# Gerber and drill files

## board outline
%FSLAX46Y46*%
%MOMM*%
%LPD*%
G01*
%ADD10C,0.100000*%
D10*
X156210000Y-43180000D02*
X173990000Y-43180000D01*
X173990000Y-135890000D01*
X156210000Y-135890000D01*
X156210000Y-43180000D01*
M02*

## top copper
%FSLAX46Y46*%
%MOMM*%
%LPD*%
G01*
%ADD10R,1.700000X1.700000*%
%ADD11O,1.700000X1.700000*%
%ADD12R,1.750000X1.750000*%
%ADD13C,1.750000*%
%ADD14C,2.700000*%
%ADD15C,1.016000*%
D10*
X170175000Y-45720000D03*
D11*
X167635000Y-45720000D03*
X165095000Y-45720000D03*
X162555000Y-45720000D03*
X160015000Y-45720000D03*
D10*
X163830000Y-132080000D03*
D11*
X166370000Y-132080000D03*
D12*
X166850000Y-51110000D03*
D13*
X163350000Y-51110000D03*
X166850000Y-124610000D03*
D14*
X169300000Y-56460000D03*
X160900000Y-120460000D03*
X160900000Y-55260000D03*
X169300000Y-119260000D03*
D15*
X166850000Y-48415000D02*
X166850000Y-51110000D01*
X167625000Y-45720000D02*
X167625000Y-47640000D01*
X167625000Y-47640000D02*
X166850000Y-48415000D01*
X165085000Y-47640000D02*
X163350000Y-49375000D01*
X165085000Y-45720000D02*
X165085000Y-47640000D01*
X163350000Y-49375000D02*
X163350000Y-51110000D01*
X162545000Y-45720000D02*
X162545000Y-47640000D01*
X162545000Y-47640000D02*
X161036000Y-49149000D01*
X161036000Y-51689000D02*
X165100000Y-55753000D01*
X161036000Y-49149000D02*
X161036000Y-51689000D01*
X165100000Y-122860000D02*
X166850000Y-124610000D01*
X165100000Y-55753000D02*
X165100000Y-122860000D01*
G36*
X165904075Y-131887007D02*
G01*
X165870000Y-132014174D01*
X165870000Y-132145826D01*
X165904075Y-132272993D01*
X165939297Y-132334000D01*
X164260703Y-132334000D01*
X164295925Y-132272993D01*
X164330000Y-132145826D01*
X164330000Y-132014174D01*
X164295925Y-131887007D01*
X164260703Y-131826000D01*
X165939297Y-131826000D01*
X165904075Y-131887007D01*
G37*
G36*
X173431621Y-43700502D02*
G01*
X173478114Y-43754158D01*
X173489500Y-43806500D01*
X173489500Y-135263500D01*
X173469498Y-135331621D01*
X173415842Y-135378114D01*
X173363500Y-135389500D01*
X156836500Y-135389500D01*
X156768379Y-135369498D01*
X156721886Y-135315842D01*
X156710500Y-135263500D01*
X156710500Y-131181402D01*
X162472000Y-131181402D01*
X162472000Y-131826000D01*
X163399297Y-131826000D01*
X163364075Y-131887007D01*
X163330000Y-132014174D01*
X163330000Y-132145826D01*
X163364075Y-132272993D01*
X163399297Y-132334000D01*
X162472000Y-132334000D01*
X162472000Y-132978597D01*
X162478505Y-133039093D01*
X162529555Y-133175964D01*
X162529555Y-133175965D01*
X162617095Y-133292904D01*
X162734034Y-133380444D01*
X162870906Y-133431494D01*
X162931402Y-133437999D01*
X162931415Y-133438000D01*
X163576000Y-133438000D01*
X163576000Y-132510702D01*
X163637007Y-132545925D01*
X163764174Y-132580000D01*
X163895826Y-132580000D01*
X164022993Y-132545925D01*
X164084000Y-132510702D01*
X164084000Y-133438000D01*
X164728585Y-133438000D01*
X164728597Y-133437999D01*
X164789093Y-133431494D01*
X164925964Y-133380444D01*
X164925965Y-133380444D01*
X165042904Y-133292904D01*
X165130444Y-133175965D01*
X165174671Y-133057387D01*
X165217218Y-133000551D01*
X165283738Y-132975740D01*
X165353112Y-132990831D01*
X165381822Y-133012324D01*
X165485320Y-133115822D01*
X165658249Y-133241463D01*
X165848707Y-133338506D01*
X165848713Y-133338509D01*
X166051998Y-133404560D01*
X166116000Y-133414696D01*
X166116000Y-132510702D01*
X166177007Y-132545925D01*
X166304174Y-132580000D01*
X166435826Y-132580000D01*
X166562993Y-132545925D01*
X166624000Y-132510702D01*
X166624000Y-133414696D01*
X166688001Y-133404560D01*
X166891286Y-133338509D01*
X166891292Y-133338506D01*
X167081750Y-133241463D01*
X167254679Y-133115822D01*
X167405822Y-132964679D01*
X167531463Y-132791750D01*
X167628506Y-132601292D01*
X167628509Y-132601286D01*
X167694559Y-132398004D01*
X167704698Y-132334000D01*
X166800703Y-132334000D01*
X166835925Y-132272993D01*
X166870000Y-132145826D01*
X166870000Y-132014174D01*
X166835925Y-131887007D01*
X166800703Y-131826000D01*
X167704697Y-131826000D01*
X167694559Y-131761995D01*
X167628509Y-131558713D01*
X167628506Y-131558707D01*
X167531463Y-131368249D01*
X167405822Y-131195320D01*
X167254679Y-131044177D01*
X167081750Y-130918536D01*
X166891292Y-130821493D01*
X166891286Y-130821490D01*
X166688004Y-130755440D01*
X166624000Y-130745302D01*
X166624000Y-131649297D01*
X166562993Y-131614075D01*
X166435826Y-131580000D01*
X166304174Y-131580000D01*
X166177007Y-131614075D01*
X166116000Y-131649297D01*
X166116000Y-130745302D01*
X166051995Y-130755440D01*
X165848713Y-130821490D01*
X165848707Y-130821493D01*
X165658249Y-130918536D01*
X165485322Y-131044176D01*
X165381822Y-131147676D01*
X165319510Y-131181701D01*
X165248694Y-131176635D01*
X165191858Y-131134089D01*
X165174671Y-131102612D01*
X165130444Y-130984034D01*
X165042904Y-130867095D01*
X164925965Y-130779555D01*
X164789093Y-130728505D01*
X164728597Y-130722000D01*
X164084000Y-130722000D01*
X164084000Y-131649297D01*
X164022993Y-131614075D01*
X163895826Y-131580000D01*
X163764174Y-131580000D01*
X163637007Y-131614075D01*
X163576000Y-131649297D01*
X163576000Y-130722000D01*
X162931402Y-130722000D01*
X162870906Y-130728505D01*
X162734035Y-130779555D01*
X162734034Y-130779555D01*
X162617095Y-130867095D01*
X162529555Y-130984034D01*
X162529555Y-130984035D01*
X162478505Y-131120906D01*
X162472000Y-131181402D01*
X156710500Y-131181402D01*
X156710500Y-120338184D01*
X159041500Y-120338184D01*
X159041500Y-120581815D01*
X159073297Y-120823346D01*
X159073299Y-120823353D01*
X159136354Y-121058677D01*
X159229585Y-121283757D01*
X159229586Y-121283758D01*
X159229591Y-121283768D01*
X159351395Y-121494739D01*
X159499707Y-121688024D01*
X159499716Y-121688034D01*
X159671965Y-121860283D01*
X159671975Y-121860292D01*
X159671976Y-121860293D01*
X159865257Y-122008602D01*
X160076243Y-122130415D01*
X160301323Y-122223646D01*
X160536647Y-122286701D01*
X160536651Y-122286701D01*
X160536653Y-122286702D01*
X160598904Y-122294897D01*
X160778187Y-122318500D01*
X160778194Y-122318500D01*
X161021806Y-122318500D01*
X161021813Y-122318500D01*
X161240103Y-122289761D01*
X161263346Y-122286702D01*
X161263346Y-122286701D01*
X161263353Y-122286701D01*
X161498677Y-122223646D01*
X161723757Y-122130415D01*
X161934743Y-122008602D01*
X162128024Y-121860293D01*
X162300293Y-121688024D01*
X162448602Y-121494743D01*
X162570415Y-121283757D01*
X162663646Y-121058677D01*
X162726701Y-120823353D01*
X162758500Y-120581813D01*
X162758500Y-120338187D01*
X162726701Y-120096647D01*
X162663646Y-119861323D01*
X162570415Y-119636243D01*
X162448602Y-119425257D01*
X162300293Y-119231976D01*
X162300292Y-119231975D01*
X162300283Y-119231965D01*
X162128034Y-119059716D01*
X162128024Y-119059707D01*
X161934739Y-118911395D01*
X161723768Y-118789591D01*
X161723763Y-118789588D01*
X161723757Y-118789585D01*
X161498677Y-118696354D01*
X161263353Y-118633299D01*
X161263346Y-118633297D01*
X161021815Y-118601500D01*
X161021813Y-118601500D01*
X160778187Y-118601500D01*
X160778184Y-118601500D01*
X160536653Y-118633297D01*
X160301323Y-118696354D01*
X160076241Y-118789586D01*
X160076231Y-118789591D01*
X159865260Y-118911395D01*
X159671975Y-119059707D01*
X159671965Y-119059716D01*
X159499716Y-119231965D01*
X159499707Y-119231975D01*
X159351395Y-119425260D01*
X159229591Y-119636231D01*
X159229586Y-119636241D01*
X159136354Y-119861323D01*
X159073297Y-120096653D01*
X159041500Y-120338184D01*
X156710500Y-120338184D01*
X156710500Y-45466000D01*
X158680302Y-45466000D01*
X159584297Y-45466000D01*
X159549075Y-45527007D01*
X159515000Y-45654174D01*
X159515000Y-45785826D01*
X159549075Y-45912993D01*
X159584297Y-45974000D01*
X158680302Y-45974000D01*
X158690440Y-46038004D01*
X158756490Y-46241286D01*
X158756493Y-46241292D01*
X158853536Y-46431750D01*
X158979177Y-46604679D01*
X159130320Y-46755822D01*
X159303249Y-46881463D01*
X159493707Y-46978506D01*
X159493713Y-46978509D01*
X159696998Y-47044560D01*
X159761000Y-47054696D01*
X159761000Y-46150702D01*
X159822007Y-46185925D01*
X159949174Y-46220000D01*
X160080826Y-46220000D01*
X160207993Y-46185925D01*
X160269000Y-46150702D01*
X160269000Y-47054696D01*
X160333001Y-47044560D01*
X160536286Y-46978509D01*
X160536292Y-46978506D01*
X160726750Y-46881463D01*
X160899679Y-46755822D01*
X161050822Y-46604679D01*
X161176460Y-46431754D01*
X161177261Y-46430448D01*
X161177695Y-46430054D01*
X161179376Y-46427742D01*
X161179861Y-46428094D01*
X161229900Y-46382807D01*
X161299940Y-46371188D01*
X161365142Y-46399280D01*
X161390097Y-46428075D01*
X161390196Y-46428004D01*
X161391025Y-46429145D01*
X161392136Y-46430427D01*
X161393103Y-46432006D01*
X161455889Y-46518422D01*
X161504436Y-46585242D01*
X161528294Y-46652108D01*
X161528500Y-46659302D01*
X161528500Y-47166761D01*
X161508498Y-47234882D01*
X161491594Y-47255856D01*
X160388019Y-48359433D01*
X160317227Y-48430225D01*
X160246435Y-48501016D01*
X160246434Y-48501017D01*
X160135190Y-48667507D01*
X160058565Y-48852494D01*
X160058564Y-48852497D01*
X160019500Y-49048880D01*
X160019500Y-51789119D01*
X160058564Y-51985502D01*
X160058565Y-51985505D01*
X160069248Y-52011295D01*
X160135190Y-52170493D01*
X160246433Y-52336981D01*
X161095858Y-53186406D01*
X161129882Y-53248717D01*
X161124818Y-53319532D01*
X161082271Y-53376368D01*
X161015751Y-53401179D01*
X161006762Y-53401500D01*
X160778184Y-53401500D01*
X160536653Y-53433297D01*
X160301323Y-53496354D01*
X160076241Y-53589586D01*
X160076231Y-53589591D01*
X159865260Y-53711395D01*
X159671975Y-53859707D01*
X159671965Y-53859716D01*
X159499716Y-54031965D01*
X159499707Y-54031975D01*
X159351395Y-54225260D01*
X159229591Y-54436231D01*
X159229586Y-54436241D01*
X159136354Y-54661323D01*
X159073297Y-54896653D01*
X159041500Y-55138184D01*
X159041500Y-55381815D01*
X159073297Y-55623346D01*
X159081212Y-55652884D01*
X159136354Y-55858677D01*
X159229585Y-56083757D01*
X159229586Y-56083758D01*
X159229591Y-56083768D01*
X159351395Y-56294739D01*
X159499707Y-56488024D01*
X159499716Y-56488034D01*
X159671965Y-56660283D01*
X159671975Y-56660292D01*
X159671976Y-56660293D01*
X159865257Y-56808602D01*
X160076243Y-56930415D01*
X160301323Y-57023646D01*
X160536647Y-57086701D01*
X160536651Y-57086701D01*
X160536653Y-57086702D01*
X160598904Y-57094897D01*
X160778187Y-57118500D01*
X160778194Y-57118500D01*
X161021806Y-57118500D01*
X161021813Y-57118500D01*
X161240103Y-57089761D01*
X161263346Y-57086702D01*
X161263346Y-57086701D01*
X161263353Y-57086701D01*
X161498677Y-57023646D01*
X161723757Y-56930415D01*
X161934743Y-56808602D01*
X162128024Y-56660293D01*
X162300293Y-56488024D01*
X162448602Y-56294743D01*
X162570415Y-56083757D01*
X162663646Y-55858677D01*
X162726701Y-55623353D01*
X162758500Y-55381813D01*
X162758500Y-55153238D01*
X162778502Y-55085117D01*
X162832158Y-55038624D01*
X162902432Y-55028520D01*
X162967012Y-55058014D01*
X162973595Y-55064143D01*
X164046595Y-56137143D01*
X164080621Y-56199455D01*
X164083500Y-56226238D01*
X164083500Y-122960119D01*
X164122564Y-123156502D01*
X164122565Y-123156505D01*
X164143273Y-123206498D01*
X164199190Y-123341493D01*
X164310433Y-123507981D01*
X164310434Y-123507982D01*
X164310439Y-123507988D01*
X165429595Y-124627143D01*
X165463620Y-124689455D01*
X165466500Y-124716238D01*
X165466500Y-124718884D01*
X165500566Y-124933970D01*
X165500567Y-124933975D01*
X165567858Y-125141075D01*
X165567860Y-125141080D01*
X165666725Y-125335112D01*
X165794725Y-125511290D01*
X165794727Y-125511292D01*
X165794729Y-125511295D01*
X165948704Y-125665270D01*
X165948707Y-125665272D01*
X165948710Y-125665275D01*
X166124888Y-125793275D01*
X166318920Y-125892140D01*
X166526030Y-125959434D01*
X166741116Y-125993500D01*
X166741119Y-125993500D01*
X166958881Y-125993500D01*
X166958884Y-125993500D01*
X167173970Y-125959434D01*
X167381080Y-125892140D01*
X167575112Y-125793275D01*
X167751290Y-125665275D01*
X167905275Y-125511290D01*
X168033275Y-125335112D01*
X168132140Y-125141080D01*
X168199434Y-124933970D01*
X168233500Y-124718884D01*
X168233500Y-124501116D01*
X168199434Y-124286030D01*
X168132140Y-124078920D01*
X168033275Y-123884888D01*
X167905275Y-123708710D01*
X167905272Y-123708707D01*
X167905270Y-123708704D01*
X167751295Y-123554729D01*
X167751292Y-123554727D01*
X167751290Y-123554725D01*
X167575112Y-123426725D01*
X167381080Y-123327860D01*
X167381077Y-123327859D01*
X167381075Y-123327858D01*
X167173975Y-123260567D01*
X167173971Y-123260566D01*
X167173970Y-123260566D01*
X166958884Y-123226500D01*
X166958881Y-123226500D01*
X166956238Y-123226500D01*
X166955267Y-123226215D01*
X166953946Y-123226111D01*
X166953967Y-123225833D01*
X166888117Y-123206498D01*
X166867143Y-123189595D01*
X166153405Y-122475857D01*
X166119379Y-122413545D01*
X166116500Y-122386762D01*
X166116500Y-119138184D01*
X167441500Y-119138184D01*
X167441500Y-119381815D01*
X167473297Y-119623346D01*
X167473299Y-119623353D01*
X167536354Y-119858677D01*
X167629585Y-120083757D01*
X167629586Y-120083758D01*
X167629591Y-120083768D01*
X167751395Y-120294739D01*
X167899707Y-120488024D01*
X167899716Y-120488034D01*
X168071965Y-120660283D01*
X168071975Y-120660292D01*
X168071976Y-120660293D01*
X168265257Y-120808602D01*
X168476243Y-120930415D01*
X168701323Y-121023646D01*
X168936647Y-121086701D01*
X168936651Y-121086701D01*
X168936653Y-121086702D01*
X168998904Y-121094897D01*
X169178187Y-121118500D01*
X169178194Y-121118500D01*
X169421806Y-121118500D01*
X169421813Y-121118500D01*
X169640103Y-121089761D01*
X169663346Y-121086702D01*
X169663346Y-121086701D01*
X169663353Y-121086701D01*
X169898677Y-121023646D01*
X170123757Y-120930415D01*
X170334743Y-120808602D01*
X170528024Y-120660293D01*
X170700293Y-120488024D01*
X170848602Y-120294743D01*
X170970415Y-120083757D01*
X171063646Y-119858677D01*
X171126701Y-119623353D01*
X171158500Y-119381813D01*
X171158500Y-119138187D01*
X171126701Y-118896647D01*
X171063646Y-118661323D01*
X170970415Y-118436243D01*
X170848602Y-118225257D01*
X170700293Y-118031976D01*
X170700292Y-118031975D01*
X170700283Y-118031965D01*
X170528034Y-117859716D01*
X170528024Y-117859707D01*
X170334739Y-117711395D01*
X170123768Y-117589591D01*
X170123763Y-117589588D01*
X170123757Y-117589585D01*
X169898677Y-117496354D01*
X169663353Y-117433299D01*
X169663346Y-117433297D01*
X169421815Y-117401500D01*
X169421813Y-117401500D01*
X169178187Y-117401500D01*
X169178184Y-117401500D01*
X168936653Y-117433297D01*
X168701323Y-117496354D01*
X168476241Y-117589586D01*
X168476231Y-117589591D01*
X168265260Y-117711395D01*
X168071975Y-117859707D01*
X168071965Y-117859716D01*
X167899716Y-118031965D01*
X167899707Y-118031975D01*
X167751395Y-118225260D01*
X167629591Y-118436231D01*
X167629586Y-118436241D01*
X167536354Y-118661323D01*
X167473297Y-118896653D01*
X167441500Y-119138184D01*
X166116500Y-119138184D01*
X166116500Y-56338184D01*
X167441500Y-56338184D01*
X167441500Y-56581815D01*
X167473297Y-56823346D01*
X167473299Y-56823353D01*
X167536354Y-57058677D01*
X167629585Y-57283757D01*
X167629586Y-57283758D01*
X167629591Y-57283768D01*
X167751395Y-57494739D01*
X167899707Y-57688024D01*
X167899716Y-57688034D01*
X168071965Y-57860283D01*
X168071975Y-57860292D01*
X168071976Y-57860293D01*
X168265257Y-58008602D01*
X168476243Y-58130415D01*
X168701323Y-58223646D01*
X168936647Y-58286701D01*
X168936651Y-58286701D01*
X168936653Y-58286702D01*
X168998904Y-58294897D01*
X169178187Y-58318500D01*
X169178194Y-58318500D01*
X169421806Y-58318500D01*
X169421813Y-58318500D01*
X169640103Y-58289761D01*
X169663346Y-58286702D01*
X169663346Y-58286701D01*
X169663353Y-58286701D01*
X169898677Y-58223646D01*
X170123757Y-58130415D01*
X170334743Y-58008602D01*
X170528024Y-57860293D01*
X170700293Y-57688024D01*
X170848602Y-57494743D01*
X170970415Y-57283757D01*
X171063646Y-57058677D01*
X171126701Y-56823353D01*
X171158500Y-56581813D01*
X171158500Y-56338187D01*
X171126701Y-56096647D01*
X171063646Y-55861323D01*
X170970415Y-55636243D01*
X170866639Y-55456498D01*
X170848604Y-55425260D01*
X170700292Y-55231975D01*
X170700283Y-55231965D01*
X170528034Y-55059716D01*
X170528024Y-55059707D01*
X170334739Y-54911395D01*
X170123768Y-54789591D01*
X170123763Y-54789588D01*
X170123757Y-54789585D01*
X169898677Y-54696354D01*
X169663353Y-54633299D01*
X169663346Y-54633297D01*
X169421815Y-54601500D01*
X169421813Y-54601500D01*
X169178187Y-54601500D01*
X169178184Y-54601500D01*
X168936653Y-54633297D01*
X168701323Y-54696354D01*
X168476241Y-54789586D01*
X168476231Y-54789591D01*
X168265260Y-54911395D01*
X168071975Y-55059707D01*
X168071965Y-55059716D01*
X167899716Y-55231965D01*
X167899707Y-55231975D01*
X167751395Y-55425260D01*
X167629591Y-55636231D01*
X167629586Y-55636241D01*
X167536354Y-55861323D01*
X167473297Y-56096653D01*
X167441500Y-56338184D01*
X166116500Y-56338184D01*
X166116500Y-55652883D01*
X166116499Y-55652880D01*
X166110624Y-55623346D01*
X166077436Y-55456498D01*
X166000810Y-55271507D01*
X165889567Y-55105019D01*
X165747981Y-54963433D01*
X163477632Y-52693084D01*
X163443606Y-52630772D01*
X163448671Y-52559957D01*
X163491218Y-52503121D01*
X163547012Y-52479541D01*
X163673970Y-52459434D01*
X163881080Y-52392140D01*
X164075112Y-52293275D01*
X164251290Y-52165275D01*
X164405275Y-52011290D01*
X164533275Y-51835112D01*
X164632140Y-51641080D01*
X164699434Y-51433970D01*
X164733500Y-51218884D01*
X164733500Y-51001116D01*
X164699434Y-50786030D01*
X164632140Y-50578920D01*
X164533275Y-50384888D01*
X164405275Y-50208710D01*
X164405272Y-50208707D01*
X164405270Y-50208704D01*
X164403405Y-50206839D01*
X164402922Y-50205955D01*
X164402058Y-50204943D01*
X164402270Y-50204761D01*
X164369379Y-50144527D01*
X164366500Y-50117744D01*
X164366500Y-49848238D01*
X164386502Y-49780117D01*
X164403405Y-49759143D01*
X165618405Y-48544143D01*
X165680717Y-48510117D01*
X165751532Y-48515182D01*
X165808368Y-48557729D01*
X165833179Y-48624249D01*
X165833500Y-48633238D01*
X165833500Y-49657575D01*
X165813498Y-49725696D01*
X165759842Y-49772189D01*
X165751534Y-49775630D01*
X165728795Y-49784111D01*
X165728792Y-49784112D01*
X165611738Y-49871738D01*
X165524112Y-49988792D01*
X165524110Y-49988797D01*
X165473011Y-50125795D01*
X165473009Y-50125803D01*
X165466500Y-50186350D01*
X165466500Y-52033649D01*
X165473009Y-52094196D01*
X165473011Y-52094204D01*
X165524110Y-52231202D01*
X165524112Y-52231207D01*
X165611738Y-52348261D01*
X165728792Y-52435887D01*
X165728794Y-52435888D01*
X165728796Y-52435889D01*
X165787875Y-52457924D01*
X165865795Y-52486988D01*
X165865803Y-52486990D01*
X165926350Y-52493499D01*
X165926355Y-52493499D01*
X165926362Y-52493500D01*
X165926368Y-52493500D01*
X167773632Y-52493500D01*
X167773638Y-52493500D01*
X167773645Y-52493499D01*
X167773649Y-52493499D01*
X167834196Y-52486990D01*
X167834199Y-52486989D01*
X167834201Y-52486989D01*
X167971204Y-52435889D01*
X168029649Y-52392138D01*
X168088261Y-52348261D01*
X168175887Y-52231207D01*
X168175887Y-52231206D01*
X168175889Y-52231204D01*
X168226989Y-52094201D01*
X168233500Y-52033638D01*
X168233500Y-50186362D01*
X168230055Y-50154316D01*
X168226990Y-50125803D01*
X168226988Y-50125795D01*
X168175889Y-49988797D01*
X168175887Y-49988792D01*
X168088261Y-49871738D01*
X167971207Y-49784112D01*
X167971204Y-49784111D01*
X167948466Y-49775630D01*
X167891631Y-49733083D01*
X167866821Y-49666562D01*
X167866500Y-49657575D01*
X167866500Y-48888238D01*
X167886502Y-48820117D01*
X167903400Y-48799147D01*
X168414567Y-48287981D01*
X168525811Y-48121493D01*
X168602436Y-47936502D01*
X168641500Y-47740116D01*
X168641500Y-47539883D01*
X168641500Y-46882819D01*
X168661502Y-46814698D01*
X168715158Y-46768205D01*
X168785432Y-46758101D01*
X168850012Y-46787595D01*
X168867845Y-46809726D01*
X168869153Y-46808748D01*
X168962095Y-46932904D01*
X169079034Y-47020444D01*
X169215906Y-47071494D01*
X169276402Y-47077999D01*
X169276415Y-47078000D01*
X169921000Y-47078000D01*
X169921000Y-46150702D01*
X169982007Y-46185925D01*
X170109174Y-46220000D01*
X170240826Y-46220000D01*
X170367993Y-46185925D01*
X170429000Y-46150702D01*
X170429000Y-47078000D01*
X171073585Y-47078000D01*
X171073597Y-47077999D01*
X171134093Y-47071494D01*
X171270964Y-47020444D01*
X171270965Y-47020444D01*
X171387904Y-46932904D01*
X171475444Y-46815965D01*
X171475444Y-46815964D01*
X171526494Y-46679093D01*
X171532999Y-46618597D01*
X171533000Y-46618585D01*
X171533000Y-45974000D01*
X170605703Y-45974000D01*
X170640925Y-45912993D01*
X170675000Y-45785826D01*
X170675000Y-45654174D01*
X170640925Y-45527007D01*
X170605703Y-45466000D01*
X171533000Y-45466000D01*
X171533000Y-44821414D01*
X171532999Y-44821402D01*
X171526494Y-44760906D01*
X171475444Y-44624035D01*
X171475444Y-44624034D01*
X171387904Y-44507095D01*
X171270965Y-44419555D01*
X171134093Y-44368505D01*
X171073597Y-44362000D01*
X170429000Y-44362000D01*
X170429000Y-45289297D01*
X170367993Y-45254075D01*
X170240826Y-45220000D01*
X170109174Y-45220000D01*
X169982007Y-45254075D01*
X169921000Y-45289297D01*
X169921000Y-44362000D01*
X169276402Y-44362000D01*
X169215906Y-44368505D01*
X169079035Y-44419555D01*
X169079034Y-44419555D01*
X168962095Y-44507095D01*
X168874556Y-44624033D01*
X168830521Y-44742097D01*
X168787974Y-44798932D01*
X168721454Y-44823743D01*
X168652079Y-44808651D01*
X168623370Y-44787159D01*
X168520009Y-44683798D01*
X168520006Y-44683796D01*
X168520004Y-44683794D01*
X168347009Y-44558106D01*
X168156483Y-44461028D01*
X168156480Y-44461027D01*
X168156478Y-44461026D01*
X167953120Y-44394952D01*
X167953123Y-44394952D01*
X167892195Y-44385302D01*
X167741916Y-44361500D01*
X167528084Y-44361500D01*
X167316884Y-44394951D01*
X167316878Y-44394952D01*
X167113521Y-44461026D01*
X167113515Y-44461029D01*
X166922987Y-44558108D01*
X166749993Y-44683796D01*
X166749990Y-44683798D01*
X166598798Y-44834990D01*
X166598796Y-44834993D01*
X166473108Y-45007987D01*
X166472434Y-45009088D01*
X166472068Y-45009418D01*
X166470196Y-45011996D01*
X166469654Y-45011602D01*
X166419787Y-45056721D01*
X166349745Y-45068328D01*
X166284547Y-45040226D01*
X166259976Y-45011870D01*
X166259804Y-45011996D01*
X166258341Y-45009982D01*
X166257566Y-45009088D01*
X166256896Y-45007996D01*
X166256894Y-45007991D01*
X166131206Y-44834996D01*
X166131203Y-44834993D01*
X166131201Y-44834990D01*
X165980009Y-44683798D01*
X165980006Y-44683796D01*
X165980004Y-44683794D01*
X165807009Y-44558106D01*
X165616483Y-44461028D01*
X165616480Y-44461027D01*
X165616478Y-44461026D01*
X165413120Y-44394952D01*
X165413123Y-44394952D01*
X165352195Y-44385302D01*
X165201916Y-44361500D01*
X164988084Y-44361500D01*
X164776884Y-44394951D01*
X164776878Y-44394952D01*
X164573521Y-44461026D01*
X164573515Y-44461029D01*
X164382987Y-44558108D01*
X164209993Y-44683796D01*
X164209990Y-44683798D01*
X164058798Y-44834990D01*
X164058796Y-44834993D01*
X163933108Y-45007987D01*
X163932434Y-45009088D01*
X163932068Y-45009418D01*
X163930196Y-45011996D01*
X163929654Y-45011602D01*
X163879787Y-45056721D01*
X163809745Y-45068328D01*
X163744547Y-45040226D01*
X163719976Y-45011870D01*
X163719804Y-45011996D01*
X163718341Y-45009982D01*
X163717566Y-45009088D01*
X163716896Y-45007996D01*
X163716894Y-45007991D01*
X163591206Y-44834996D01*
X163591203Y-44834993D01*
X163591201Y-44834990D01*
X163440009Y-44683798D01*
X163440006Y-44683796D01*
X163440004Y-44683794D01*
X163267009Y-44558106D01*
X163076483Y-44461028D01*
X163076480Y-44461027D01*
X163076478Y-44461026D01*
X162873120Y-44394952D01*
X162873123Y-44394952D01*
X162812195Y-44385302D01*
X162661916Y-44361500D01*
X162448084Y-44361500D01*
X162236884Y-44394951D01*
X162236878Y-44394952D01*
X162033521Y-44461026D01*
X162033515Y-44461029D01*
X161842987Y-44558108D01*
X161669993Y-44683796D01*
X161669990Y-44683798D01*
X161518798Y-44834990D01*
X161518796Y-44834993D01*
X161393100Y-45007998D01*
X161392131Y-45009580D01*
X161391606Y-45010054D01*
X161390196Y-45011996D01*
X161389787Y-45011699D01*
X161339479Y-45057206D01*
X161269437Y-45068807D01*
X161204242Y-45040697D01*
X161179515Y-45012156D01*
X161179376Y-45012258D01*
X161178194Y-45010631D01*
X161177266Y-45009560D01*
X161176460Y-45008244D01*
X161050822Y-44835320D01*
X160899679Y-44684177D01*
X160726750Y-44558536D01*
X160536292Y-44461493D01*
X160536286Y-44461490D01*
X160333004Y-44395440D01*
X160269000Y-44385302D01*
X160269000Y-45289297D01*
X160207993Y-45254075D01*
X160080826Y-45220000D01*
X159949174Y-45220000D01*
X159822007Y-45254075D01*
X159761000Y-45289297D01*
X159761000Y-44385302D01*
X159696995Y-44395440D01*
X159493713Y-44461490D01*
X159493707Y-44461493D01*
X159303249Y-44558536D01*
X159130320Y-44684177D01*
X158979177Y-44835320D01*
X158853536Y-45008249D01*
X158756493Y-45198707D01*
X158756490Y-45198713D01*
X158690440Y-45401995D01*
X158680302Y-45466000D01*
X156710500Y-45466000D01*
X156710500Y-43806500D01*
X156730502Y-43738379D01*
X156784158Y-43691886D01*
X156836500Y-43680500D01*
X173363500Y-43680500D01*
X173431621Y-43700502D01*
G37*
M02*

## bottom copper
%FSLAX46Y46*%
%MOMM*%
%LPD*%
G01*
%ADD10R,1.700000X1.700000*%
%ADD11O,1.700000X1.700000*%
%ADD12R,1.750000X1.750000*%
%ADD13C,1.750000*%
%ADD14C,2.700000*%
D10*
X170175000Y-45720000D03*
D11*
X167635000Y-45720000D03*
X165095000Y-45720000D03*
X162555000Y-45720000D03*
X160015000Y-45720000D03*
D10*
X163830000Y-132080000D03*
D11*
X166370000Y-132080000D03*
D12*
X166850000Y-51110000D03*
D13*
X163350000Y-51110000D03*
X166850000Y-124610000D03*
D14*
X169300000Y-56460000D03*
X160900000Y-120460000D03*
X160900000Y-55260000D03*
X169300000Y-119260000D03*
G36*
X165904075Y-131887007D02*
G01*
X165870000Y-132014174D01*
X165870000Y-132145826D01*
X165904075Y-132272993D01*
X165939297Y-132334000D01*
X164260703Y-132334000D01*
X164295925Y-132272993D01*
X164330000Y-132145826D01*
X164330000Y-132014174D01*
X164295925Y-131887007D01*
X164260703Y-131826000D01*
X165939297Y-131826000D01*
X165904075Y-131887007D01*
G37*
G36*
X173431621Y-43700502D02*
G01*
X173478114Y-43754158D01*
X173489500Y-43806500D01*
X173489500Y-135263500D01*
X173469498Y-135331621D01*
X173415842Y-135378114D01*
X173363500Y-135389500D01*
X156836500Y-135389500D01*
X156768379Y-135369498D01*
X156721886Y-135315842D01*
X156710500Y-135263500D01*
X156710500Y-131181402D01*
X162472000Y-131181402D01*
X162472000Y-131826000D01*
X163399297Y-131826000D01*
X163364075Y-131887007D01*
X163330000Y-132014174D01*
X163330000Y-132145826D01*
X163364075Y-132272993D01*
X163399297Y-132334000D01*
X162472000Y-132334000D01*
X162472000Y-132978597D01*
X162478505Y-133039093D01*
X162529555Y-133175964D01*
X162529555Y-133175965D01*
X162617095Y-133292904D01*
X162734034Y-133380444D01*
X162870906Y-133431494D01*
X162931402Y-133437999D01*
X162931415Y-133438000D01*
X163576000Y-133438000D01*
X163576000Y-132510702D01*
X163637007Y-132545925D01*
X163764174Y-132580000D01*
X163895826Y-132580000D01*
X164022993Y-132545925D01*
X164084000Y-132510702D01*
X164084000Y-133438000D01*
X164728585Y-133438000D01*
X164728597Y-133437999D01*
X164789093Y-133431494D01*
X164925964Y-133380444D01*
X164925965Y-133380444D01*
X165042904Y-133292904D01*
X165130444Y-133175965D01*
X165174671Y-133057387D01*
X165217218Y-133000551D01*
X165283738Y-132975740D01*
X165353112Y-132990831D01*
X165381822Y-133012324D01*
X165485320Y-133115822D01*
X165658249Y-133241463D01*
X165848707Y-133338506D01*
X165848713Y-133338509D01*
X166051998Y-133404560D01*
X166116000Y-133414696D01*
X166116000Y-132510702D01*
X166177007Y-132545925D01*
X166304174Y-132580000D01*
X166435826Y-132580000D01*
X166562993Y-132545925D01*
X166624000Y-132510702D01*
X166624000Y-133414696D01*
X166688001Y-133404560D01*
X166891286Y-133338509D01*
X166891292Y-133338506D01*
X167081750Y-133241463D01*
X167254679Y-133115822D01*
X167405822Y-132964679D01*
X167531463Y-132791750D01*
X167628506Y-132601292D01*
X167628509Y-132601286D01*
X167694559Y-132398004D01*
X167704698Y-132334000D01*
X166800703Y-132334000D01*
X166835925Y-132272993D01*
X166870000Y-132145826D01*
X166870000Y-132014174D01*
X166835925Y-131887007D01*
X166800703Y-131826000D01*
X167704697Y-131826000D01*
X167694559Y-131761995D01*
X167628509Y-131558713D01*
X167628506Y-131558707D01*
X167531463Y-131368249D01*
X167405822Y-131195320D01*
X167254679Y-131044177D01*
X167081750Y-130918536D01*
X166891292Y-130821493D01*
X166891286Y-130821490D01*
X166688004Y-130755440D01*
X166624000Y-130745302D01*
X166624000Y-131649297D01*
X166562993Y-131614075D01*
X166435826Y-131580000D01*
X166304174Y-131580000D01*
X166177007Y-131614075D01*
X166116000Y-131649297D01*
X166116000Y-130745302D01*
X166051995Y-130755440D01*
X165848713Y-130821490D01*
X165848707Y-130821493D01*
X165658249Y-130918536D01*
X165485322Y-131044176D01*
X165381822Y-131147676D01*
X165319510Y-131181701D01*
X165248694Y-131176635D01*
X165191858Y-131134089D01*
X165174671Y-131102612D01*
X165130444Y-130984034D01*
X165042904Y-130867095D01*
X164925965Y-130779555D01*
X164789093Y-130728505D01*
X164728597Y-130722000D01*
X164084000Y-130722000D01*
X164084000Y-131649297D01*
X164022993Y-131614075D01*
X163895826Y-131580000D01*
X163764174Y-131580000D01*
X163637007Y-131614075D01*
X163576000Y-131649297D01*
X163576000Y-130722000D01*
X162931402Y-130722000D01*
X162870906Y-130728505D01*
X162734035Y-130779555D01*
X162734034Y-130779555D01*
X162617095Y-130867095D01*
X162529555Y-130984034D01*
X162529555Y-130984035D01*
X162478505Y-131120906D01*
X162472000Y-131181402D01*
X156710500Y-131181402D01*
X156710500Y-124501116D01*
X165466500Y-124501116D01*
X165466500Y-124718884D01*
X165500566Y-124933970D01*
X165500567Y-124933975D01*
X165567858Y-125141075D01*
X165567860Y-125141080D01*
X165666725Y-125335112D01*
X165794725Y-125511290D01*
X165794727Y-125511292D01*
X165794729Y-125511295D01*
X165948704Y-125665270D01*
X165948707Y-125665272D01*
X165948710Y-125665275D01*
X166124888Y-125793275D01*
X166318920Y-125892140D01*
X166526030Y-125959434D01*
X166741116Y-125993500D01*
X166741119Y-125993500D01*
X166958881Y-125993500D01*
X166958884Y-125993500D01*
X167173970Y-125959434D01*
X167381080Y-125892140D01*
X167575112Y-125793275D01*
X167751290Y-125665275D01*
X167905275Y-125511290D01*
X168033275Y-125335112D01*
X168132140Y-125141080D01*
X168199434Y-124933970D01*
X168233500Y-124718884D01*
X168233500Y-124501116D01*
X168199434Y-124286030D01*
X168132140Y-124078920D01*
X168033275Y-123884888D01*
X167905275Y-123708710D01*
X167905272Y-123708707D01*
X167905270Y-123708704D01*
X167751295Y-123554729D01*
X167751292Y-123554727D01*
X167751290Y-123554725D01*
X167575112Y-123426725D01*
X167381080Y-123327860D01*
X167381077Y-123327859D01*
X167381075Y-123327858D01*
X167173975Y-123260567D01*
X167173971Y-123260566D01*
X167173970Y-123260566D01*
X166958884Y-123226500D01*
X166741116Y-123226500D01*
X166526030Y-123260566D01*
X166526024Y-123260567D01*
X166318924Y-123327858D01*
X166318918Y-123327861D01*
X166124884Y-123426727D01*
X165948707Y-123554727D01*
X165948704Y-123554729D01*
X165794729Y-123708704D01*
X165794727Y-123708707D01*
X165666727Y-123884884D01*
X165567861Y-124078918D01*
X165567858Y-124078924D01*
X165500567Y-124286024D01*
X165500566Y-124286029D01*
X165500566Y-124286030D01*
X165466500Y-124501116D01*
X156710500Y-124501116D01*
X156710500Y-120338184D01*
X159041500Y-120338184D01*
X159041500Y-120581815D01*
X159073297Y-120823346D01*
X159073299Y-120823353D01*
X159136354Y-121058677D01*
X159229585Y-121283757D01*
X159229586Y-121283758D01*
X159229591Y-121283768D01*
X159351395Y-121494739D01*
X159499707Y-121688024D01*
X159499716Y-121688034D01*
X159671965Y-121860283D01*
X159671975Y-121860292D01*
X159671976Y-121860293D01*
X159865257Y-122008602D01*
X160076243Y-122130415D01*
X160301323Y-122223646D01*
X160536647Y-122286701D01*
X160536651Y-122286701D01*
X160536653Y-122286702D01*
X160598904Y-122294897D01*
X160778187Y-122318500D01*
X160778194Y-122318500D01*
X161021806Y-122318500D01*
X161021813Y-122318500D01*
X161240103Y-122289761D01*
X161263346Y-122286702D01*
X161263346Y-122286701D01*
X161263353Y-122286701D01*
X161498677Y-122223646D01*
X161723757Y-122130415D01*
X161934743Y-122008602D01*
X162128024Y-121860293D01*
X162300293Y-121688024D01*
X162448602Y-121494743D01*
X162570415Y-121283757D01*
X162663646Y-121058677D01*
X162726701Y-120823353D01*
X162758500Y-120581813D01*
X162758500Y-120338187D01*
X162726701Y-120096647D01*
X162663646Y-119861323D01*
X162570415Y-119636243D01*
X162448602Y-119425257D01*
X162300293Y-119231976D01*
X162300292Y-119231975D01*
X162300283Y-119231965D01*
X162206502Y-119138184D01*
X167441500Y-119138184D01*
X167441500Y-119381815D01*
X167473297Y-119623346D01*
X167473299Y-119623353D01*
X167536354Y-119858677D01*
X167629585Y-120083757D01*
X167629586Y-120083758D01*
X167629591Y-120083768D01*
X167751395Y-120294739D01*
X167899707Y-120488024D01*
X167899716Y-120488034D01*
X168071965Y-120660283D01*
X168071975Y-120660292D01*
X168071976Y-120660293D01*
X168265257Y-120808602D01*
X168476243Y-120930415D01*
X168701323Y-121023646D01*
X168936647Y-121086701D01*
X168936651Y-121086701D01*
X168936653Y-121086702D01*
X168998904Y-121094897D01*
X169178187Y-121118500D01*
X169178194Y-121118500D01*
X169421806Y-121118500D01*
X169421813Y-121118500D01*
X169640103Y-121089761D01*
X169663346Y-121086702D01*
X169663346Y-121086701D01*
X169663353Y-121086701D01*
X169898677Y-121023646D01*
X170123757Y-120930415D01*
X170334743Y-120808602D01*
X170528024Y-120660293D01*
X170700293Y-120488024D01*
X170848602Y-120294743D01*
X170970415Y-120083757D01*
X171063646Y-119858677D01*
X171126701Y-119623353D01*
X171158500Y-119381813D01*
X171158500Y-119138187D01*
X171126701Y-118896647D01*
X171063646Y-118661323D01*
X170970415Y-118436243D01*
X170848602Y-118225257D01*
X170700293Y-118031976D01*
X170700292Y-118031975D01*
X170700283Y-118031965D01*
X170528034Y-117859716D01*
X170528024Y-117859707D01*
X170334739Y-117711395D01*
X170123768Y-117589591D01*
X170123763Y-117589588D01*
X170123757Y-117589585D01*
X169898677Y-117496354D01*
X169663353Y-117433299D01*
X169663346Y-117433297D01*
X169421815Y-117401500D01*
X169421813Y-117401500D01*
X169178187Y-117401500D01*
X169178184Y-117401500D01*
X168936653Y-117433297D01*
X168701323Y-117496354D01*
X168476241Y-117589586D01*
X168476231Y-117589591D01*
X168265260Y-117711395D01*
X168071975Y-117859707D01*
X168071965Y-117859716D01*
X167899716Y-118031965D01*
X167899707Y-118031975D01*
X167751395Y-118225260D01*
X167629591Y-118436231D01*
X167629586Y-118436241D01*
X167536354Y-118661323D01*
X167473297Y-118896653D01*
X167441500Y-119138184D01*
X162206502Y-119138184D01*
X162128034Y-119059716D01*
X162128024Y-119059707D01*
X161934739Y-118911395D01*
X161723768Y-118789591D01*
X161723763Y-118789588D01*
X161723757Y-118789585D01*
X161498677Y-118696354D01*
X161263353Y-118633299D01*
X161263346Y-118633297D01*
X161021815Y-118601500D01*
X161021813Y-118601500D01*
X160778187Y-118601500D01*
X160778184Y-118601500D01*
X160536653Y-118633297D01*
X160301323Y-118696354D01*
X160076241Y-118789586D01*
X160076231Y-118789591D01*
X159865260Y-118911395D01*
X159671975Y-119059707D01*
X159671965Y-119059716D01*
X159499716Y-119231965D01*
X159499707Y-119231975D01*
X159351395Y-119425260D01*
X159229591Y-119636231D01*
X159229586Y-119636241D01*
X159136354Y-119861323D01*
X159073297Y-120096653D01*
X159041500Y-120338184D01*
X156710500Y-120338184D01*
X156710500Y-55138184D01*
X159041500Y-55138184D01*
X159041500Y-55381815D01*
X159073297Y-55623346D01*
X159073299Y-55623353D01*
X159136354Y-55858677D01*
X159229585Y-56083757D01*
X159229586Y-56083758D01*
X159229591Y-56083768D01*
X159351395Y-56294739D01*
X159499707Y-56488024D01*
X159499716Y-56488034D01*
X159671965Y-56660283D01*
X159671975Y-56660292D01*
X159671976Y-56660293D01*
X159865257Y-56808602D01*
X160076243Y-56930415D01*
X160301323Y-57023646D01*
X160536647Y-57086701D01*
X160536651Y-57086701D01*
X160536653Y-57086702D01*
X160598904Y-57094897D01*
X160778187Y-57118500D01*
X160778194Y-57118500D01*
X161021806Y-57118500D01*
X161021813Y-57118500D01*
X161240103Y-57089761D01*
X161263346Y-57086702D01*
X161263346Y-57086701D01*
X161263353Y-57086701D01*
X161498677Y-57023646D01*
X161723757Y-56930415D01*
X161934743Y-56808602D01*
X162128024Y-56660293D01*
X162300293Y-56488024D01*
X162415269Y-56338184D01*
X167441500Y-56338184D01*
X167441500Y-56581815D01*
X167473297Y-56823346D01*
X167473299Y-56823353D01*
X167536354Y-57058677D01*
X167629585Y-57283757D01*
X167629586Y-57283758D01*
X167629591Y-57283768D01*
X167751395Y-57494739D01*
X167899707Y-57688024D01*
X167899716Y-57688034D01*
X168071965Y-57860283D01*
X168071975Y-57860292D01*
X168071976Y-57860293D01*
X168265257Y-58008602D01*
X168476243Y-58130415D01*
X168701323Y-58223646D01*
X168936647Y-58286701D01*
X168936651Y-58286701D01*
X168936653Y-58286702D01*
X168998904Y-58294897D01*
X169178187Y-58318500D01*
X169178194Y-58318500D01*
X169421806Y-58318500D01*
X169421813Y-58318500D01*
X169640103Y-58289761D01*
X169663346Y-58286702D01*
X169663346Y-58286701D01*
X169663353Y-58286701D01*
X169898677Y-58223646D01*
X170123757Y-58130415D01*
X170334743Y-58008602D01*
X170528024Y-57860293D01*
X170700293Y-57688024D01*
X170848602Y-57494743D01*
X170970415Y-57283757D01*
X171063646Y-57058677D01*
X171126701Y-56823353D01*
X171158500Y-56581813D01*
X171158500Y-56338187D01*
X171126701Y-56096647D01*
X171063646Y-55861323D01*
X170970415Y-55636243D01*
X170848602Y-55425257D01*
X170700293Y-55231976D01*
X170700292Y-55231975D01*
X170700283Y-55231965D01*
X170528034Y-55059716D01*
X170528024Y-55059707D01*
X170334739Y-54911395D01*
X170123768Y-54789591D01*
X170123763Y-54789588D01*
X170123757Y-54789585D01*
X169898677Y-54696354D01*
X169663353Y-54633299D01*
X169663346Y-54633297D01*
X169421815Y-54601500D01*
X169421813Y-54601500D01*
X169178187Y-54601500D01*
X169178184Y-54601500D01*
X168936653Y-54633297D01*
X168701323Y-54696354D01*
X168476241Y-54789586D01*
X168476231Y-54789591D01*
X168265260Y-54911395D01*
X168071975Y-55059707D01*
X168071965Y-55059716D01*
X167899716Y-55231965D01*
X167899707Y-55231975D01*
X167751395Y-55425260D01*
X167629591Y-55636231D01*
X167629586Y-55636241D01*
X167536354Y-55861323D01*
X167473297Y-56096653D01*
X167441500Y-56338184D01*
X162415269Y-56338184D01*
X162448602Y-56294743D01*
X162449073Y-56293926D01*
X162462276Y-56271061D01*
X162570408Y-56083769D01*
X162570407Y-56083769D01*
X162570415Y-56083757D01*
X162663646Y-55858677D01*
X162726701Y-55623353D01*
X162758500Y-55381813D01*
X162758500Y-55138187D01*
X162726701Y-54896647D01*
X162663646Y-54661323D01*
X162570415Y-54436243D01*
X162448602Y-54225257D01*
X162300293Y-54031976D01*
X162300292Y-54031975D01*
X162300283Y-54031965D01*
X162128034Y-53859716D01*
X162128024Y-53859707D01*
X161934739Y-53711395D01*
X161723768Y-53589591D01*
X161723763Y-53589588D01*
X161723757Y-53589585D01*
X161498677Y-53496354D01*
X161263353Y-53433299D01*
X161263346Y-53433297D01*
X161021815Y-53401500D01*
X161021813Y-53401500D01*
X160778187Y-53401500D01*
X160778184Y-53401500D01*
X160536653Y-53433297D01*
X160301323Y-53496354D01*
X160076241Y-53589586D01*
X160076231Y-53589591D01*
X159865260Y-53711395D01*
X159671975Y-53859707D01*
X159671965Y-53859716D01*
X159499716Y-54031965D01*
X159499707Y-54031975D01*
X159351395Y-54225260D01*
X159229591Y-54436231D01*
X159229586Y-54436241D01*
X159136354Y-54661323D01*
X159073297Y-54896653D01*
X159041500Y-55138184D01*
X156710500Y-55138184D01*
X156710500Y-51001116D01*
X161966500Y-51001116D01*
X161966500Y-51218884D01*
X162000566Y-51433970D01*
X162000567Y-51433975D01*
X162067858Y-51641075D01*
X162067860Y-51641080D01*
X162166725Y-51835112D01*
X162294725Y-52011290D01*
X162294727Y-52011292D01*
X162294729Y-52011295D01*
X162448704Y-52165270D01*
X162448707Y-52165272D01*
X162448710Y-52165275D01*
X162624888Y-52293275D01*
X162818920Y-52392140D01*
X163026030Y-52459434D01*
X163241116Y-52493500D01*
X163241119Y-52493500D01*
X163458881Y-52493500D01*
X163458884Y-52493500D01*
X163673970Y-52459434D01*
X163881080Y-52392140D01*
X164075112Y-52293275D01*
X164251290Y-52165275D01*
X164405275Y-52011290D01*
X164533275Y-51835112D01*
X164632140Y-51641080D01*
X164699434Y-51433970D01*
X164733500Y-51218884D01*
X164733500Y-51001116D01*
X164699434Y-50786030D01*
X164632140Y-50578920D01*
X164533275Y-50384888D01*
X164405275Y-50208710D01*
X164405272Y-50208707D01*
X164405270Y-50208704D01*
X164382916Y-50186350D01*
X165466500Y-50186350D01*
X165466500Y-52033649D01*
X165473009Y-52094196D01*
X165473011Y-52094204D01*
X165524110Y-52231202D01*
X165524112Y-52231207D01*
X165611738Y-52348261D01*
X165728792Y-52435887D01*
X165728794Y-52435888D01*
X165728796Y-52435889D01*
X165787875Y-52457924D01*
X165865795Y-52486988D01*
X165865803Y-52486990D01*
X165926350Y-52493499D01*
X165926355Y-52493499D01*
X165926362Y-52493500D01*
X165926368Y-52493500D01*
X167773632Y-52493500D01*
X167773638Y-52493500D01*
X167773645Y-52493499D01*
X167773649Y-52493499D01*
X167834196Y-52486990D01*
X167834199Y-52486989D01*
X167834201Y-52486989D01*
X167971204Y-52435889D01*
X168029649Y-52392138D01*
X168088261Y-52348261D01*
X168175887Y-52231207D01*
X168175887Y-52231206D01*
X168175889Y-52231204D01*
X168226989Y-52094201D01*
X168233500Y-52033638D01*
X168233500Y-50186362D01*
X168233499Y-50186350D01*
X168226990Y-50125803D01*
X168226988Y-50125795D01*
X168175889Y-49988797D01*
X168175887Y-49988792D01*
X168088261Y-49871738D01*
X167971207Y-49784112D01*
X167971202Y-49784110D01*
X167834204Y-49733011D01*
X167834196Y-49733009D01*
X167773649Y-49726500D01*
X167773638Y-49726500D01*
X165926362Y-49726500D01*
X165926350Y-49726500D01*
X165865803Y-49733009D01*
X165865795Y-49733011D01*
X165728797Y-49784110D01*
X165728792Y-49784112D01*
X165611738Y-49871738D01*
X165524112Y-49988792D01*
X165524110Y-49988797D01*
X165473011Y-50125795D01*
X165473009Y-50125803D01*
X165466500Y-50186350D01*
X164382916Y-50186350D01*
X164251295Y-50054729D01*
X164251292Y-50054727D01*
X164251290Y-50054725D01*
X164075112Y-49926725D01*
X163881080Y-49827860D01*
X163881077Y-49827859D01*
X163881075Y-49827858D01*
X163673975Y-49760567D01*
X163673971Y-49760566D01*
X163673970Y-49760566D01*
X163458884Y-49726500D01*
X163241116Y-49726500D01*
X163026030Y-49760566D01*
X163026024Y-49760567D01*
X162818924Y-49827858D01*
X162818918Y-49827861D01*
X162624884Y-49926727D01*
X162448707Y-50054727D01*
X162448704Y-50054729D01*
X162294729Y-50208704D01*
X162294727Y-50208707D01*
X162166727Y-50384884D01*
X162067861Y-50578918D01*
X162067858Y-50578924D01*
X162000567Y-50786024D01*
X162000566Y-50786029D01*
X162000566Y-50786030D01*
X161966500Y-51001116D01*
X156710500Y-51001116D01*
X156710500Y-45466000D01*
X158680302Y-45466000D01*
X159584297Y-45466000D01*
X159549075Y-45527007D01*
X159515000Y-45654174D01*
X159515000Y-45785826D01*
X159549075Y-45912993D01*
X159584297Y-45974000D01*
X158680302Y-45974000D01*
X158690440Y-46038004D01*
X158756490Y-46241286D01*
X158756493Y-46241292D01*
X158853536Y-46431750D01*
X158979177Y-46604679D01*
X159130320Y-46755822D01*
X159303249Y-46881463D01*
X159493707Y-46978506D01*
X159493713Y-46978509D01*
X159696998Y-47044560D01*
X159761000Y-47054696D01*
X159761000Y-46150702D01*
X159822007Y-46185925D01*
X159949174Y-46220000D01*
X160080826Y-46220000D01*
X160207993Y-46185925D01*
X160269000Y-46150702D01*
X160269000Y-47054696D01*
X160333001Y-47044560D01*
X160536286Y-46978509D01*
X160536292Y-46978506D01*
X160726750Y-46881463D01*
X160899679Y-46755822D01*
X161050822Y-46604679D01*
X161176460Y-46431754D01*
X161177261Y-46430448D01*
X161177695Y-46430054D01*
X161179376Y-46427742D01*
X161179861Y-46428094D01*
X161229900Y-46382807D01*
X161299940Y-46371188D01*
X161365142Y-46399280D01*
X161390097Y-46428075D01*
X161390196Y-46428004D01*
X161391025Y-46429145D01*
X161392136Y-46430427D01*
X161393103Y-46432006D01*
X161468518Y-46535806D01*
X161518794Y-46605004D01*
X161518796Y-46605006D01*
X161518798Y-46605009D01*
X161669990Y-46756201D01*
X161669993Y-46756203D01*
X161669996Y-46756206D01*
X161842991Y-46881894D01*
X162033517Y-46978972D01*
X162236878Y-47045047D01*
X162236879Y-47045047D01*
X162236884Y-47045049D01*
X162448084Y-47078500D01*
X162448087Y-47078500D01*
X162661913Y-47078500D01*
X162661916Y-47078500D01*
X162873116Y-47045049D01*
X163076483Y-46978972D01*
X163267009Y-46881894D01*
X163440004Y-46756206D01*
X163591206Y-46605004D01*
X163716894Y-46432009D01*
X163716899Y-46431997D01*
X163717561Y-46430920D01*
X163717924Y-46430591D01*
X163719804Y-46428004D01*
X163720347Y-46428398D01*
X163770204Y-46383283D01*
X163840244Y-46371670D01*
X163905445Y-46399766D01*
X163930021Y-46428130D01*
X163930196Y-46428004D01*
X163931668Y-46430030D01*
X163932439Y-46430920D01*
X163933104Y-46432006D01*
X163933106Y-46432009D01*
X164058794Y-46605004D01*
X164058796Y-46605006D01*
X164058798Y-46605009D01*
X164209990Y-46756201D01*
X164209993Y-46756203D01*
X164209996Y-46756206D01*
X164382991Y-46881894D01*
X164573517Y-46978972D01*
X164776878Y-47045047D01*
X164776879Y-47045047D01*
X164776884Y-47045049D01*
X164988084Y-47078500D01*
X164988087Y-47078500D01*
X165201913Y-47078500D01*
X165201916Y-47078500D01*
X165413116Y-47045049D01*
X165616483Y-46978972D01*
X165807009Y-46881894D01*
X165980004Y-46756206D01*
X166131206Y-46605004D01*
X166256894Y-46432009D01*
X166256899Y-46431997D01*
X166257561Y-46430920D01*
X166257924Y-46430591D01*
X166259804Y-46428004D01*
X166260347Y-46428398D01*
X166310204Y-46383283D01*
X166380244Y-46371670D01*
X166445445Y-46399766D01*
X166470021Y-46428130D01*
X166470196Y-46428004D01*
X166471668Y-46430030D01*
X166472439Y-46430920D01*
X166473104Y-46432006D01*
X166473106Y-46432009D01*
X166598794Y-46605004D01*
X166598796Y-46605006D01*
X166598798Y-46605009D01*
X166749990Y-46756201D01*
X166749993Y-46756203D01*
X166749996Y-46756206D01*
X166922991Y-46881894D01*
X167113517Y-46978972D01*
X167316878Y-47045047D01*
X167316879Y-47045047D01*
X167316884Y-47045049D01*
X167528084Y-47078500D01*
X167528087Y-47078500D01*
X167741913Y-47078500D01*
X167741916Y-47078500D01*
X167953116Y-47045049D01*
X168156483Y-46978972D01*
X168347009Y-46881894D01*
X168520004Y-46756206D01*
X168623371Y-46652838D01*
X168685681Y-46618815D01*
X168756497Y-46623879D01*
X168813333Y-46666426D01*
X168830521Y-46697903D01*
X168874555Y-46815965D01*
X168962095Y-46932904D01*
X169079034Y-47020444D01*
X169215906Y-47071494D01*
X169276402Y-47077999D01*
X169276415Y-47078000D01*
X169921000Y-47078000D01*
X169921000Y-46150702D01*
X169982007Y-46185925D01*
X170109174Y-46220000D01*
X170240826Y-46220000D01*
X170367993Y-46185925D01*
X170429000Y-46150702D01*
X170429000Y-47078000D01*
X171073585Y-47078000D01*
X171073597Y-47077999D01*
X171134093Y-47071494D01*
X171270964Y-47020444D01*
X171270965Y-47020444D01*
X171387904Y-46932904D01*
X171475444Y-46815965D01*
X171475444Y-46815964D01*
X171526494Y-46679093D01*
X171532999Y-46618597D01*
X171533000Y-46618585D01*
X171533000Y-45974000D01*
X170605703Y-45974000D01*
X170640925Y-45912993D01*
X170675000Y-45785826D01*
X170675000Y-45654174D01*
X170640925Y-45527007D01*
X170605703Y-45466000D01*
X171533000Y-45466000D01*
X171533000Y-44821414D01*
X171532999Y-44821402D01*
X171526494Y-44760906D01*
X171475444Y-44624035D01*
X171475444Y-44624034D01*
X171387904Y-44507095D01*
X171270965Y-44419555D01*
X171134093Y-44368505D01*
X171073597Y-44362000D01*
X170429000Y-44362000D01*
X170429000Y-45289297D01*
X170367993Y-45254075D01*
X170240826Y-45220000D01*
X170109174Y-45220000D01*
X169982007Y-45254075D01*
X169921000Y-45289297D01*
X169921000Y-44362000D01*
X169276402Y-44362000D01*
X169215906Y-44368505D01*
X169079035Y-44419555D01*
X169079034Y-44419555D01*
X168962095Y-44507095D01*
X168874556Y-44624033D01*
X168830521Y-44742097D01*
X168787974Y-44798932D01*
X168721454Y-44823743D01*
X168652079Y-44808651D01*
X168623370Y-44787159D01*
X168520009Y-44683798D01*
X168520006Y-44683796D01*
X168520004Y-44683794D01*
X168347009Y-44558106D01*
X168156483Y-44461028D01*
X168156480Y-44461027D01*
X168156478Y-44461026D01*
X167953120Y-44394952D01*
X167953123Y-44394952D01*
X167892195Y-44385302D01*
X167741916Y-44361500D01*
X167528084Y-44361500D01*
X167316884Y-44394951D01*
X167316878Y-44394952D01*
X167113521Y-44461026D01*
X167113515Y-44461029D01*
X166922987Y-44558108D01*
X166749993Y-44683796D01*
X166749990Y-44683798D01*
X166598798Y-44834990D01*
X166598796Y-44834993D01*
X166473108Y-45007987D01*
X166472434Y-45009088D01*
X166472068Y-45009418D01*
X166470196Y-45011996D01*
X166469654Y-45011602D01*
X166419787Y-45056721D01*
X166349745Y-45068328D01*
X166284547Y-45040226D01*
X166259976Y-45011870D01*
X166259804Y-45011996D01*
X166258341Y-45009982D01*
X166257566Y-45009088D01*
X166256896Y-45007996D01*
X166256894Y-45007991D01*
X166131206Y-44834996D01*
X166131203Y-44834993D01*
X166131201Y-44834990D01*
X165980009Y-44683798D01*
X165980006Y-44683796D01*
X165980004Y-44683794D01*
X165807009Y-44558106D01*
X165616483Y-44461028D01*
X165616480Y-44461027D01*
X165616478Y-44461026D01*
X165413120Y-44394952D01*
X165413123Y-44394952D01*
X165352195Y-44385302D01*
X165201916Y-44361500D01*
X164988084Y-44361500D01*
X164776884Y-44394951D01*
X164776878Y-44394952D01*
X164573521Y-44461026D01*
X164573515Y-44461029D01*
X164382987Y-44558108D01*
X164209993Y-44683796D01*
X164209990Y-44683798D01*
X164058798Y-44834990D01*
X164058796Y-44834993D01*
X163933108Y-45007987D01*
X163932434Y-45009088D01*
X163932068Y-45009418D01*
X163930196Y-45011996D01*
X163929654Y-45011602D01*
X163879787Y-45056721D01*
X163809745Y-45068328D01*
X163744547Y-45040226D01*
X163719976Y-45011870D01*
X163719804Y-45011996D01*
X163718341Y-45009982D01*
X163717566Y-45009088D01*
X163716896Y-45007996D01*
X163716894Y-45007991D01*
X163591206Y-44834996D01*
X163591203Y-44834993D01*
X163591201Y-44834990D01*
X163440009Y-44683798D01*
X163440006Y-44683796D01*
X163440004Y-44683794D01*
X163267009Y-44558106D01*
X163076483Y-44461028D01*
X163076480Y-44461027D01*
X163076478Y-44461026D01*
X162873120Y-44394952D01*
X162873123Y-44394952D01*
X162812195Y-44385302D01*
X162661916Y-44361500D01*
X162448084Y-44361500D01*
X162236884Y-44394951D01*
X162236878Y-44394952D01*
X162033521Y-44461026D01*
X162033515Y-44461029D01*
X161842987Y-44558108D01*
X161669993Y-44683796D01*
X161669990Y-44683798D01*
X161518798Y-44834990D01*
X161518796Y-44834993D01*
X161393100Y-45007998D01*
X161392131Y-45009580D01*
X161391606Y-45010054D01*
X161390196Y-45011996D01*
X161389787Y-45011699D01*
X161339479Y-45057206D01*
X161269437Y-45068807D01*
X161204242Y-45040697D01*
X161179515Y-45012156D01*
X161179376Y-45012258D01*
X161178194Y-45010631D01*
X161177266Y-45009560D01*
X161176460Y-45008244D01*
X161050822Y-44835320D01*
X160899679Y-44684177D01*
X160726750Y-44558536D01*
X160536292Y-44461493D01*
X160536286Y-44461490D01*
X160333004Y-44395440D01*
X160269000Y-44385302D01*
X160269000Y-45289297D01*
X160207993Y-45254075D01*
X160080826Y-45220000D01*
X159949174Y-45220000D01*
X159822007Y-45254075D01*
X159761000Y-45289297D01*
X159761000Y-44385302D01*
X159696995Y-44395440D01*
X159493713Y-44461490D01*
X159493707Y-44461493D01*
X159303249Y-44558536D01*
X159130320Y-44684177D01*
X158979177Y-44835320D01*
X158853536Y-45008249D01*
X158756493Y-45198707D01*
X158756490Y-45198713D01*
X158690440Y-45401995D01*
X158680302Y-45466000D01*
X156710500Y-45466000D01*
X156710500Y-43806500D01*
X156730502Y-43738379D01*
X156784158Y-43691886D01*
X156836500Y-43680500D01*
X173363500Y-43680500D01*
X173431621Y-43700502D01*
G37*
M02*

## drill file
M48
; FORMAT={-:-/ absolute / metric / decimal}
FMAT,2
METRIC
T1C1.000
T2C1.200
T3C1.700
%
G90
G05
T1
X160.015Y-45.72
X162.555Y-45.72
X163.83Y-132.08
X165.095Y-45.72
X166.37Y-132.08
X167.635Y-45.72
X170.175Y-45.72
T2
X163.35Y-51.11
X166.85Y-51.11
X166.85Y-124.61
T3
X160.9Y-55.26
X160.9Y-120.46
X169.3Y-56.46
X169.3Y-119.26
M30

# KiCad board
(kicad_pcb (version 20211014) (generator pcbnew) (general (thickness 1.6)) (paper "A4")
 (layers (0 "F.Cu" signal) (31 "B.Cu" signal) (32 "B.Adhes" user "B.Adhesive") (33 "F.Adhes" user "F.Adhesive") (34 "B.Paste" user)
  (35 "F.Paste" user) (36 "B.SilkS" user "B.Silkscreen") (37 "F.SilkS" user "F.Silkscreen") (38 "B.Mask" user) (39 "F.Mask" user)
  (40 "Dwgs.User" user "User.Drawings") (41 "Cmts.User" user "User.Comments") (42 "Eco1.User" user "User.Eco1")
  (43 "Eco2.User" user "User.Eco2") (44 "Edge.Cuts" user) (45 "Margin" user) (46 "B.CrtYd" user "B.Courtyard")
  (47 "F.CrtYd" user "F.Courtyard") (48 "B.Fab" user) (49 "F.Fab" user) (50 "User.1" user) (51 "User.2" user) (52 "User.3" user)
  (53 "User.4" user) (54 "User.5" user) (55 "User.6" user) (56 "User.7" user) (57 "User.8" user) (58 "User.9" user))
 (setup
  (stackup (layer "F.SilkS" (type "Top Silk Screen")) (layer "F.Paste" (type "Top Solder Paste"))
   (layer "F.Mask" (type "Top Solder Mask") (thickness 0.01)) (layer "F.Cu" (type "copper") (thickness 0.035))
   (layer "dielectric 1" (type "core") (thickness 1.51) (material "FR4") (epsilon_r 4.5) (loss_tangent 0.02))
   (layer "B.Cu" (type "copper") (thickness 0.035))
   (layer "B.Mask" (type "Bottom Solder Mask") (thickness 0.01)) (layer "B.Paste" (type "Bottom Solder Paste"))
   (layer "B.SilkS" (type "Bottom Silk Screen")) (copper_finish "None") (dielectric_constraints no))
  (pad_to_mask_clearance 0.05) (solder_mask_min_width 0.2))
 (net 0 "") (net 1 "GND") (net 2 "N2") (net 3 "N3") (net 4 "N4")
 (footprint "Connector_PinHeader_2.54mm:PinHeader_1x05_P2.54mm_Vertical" (layer "F.Cu") (at 170.175 45.72 -90)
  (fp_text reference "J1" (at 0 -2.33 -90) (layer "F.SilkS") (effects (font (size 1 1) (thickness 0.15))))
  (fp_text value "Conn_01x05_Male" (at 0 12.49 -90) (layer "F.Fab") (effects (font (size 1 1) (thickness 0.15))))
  (pad "1" thru_hole rect (at 0 0 270) (size 1.7 1.7) (drill 1) (layers *.Cu *.Mask) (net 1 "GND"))
  (pad "2" thru_hole oval (at 0 2.54 270) (size 1.7 1.7) (drill 1) (layers *.Cu *.Mask) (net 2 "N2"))
  (pad "3" thru_hole oval (at 0 5.08 270) (size 1.7 1.7) (drill 1) (layers *.Cu *.Mask) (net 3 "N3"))
  (pad "4" thru_hole oval (at 0 7.62 270) (size 1.7 1.7) (drill 1) (layers *.Cu *.Mask) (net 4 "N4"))
  (pad "5" thru_hole oval (at 0 10.16 270) (size 1.7 1.7) (drill 1) (layers *.Cu *.Mask) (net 1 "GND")))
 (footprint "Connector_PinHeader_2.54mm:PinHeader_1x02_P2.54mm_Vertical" (layer "F.Cu") (at 163.83 132.08 90)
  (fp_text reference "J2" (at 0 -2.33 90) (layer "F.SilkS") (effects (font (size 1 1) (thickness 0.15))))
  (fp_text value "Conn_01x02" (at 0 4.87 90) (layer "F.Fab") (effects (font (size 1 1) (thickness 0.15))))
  (pad "1" thru_hole rect (at 0 0 90) (size 1.7 1.7) (drill 1) (layers *.Cu *.Mask) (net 1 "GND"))
  (pad "2" thru_hole oval (at 0 2.54 90) (size 1.7 1.7) (drill 1) (layers *.Cu *.Mask) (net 1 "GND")))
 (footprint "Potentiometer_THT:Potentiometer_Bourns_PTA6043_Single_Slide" (layer "F.Cu") (at 166.85 51.11 -90)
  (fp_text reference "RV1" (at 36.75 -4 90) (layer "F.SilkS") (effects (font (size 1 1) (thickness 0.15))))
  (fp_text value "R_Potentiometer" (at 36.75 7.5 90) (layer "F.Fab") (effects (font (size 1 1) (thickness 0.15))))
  (pad "1" thru_hole rect (at 0 0 270) (size 1.75 1.75) (drill 1.2) (layers *.Cu *.Mask) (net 2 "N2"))
  (pad "2" thru_hole circle (at 0 3.5 270) (size 1.75 1.75) (drill 1.2) (layers *.Cu *.Mask) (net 3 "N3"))
  (pad "3" thru_hole circle (at 73.5 0 270) (size 1.75 1.75) (drill 1.2) (layers *.Cu *.Mask) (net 4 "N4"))
  (pad "MP" thru_hole circle (at 5.35 -2.45 270) (size 2.7 2.7) (drill 1.7) (layers *.Cu *.Mask))
  (pad "MP" thru_hole circle (at 69.35 5.95 270) (size 2.7 2.7) (drill 1.7) (layers *.Cu *.Mask))
  (pad "MP" thru_hole circle (at 4.15 5.95 270) (size 2.7 2.7) (drill 1.7) (layers *.Cu *.Mask))
  (pad "MP" thru_hole circle (at 68.15 -2.45 270) (size 2.7 2.7) (drill 1.7) (layers *.Cu *.Mask)))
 (gr_rect (start 156.21 43.18) (end 173.99 135.89) (layer "Edge.Cuts") (width 0.1) (fill none))
 (segment (start 166.85 48.415) (end 166.85 51.11) (width 1.016) (layer "F.Cu") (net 2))
 (segment (start 167.625 45.72) (end 167.625 47.64) (width 1.016) (layer "F.Cu") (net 2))
 (segment (start 167.625 47.64) (end 166.85 48.415) (width 1.016) (layer "F.Cu") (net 2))
 (segment (start 165.085 47.64) (end 163.35 49.375) (width 1.016) (layer "F.Cu") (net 3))
 (segment (start 165.085 45.72) (end 165.085 47.64) (width 1.016) (layer "F.Cu") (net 3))
 (segment (start 163.35 49.375) (end 163.35 51.11) (width 1.016) (layer "F.Cu") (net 3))
 (segment (start 162.545 45.72) (end 162.545 47.64) (width 1.016) (layer "F.Cu") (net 4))
 (segment (start 162.545 47.64) (end 161.036 49.149) (width 1.016) (layer "F.Cu") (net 4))
 (segment (start 161.036 51.689) (end 165.1 55.753) (width 1.016) (layer "F.Cu") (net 4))
 (segment (start 161.036 49.149) (end 161.036 51.689) (width 1.016) (layer "F.Cu") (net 4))
 (segment (start 165.1 122.86) (end 166.85 124.61) (width 1.016) (layer "F.Cu") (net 4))
 (segment (start 165.1 55.753) (end 165.1 122.86) (width 1.016) (layer "F.Cu") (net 4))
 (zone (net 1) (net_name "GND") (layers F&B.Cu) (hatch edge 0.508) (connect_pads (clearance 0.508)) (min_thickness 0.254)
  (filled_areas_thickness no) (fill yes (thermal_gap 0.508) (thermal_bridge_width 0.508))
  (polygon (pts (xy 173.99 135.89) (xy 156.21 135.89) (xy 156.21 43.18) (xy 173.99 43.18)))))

